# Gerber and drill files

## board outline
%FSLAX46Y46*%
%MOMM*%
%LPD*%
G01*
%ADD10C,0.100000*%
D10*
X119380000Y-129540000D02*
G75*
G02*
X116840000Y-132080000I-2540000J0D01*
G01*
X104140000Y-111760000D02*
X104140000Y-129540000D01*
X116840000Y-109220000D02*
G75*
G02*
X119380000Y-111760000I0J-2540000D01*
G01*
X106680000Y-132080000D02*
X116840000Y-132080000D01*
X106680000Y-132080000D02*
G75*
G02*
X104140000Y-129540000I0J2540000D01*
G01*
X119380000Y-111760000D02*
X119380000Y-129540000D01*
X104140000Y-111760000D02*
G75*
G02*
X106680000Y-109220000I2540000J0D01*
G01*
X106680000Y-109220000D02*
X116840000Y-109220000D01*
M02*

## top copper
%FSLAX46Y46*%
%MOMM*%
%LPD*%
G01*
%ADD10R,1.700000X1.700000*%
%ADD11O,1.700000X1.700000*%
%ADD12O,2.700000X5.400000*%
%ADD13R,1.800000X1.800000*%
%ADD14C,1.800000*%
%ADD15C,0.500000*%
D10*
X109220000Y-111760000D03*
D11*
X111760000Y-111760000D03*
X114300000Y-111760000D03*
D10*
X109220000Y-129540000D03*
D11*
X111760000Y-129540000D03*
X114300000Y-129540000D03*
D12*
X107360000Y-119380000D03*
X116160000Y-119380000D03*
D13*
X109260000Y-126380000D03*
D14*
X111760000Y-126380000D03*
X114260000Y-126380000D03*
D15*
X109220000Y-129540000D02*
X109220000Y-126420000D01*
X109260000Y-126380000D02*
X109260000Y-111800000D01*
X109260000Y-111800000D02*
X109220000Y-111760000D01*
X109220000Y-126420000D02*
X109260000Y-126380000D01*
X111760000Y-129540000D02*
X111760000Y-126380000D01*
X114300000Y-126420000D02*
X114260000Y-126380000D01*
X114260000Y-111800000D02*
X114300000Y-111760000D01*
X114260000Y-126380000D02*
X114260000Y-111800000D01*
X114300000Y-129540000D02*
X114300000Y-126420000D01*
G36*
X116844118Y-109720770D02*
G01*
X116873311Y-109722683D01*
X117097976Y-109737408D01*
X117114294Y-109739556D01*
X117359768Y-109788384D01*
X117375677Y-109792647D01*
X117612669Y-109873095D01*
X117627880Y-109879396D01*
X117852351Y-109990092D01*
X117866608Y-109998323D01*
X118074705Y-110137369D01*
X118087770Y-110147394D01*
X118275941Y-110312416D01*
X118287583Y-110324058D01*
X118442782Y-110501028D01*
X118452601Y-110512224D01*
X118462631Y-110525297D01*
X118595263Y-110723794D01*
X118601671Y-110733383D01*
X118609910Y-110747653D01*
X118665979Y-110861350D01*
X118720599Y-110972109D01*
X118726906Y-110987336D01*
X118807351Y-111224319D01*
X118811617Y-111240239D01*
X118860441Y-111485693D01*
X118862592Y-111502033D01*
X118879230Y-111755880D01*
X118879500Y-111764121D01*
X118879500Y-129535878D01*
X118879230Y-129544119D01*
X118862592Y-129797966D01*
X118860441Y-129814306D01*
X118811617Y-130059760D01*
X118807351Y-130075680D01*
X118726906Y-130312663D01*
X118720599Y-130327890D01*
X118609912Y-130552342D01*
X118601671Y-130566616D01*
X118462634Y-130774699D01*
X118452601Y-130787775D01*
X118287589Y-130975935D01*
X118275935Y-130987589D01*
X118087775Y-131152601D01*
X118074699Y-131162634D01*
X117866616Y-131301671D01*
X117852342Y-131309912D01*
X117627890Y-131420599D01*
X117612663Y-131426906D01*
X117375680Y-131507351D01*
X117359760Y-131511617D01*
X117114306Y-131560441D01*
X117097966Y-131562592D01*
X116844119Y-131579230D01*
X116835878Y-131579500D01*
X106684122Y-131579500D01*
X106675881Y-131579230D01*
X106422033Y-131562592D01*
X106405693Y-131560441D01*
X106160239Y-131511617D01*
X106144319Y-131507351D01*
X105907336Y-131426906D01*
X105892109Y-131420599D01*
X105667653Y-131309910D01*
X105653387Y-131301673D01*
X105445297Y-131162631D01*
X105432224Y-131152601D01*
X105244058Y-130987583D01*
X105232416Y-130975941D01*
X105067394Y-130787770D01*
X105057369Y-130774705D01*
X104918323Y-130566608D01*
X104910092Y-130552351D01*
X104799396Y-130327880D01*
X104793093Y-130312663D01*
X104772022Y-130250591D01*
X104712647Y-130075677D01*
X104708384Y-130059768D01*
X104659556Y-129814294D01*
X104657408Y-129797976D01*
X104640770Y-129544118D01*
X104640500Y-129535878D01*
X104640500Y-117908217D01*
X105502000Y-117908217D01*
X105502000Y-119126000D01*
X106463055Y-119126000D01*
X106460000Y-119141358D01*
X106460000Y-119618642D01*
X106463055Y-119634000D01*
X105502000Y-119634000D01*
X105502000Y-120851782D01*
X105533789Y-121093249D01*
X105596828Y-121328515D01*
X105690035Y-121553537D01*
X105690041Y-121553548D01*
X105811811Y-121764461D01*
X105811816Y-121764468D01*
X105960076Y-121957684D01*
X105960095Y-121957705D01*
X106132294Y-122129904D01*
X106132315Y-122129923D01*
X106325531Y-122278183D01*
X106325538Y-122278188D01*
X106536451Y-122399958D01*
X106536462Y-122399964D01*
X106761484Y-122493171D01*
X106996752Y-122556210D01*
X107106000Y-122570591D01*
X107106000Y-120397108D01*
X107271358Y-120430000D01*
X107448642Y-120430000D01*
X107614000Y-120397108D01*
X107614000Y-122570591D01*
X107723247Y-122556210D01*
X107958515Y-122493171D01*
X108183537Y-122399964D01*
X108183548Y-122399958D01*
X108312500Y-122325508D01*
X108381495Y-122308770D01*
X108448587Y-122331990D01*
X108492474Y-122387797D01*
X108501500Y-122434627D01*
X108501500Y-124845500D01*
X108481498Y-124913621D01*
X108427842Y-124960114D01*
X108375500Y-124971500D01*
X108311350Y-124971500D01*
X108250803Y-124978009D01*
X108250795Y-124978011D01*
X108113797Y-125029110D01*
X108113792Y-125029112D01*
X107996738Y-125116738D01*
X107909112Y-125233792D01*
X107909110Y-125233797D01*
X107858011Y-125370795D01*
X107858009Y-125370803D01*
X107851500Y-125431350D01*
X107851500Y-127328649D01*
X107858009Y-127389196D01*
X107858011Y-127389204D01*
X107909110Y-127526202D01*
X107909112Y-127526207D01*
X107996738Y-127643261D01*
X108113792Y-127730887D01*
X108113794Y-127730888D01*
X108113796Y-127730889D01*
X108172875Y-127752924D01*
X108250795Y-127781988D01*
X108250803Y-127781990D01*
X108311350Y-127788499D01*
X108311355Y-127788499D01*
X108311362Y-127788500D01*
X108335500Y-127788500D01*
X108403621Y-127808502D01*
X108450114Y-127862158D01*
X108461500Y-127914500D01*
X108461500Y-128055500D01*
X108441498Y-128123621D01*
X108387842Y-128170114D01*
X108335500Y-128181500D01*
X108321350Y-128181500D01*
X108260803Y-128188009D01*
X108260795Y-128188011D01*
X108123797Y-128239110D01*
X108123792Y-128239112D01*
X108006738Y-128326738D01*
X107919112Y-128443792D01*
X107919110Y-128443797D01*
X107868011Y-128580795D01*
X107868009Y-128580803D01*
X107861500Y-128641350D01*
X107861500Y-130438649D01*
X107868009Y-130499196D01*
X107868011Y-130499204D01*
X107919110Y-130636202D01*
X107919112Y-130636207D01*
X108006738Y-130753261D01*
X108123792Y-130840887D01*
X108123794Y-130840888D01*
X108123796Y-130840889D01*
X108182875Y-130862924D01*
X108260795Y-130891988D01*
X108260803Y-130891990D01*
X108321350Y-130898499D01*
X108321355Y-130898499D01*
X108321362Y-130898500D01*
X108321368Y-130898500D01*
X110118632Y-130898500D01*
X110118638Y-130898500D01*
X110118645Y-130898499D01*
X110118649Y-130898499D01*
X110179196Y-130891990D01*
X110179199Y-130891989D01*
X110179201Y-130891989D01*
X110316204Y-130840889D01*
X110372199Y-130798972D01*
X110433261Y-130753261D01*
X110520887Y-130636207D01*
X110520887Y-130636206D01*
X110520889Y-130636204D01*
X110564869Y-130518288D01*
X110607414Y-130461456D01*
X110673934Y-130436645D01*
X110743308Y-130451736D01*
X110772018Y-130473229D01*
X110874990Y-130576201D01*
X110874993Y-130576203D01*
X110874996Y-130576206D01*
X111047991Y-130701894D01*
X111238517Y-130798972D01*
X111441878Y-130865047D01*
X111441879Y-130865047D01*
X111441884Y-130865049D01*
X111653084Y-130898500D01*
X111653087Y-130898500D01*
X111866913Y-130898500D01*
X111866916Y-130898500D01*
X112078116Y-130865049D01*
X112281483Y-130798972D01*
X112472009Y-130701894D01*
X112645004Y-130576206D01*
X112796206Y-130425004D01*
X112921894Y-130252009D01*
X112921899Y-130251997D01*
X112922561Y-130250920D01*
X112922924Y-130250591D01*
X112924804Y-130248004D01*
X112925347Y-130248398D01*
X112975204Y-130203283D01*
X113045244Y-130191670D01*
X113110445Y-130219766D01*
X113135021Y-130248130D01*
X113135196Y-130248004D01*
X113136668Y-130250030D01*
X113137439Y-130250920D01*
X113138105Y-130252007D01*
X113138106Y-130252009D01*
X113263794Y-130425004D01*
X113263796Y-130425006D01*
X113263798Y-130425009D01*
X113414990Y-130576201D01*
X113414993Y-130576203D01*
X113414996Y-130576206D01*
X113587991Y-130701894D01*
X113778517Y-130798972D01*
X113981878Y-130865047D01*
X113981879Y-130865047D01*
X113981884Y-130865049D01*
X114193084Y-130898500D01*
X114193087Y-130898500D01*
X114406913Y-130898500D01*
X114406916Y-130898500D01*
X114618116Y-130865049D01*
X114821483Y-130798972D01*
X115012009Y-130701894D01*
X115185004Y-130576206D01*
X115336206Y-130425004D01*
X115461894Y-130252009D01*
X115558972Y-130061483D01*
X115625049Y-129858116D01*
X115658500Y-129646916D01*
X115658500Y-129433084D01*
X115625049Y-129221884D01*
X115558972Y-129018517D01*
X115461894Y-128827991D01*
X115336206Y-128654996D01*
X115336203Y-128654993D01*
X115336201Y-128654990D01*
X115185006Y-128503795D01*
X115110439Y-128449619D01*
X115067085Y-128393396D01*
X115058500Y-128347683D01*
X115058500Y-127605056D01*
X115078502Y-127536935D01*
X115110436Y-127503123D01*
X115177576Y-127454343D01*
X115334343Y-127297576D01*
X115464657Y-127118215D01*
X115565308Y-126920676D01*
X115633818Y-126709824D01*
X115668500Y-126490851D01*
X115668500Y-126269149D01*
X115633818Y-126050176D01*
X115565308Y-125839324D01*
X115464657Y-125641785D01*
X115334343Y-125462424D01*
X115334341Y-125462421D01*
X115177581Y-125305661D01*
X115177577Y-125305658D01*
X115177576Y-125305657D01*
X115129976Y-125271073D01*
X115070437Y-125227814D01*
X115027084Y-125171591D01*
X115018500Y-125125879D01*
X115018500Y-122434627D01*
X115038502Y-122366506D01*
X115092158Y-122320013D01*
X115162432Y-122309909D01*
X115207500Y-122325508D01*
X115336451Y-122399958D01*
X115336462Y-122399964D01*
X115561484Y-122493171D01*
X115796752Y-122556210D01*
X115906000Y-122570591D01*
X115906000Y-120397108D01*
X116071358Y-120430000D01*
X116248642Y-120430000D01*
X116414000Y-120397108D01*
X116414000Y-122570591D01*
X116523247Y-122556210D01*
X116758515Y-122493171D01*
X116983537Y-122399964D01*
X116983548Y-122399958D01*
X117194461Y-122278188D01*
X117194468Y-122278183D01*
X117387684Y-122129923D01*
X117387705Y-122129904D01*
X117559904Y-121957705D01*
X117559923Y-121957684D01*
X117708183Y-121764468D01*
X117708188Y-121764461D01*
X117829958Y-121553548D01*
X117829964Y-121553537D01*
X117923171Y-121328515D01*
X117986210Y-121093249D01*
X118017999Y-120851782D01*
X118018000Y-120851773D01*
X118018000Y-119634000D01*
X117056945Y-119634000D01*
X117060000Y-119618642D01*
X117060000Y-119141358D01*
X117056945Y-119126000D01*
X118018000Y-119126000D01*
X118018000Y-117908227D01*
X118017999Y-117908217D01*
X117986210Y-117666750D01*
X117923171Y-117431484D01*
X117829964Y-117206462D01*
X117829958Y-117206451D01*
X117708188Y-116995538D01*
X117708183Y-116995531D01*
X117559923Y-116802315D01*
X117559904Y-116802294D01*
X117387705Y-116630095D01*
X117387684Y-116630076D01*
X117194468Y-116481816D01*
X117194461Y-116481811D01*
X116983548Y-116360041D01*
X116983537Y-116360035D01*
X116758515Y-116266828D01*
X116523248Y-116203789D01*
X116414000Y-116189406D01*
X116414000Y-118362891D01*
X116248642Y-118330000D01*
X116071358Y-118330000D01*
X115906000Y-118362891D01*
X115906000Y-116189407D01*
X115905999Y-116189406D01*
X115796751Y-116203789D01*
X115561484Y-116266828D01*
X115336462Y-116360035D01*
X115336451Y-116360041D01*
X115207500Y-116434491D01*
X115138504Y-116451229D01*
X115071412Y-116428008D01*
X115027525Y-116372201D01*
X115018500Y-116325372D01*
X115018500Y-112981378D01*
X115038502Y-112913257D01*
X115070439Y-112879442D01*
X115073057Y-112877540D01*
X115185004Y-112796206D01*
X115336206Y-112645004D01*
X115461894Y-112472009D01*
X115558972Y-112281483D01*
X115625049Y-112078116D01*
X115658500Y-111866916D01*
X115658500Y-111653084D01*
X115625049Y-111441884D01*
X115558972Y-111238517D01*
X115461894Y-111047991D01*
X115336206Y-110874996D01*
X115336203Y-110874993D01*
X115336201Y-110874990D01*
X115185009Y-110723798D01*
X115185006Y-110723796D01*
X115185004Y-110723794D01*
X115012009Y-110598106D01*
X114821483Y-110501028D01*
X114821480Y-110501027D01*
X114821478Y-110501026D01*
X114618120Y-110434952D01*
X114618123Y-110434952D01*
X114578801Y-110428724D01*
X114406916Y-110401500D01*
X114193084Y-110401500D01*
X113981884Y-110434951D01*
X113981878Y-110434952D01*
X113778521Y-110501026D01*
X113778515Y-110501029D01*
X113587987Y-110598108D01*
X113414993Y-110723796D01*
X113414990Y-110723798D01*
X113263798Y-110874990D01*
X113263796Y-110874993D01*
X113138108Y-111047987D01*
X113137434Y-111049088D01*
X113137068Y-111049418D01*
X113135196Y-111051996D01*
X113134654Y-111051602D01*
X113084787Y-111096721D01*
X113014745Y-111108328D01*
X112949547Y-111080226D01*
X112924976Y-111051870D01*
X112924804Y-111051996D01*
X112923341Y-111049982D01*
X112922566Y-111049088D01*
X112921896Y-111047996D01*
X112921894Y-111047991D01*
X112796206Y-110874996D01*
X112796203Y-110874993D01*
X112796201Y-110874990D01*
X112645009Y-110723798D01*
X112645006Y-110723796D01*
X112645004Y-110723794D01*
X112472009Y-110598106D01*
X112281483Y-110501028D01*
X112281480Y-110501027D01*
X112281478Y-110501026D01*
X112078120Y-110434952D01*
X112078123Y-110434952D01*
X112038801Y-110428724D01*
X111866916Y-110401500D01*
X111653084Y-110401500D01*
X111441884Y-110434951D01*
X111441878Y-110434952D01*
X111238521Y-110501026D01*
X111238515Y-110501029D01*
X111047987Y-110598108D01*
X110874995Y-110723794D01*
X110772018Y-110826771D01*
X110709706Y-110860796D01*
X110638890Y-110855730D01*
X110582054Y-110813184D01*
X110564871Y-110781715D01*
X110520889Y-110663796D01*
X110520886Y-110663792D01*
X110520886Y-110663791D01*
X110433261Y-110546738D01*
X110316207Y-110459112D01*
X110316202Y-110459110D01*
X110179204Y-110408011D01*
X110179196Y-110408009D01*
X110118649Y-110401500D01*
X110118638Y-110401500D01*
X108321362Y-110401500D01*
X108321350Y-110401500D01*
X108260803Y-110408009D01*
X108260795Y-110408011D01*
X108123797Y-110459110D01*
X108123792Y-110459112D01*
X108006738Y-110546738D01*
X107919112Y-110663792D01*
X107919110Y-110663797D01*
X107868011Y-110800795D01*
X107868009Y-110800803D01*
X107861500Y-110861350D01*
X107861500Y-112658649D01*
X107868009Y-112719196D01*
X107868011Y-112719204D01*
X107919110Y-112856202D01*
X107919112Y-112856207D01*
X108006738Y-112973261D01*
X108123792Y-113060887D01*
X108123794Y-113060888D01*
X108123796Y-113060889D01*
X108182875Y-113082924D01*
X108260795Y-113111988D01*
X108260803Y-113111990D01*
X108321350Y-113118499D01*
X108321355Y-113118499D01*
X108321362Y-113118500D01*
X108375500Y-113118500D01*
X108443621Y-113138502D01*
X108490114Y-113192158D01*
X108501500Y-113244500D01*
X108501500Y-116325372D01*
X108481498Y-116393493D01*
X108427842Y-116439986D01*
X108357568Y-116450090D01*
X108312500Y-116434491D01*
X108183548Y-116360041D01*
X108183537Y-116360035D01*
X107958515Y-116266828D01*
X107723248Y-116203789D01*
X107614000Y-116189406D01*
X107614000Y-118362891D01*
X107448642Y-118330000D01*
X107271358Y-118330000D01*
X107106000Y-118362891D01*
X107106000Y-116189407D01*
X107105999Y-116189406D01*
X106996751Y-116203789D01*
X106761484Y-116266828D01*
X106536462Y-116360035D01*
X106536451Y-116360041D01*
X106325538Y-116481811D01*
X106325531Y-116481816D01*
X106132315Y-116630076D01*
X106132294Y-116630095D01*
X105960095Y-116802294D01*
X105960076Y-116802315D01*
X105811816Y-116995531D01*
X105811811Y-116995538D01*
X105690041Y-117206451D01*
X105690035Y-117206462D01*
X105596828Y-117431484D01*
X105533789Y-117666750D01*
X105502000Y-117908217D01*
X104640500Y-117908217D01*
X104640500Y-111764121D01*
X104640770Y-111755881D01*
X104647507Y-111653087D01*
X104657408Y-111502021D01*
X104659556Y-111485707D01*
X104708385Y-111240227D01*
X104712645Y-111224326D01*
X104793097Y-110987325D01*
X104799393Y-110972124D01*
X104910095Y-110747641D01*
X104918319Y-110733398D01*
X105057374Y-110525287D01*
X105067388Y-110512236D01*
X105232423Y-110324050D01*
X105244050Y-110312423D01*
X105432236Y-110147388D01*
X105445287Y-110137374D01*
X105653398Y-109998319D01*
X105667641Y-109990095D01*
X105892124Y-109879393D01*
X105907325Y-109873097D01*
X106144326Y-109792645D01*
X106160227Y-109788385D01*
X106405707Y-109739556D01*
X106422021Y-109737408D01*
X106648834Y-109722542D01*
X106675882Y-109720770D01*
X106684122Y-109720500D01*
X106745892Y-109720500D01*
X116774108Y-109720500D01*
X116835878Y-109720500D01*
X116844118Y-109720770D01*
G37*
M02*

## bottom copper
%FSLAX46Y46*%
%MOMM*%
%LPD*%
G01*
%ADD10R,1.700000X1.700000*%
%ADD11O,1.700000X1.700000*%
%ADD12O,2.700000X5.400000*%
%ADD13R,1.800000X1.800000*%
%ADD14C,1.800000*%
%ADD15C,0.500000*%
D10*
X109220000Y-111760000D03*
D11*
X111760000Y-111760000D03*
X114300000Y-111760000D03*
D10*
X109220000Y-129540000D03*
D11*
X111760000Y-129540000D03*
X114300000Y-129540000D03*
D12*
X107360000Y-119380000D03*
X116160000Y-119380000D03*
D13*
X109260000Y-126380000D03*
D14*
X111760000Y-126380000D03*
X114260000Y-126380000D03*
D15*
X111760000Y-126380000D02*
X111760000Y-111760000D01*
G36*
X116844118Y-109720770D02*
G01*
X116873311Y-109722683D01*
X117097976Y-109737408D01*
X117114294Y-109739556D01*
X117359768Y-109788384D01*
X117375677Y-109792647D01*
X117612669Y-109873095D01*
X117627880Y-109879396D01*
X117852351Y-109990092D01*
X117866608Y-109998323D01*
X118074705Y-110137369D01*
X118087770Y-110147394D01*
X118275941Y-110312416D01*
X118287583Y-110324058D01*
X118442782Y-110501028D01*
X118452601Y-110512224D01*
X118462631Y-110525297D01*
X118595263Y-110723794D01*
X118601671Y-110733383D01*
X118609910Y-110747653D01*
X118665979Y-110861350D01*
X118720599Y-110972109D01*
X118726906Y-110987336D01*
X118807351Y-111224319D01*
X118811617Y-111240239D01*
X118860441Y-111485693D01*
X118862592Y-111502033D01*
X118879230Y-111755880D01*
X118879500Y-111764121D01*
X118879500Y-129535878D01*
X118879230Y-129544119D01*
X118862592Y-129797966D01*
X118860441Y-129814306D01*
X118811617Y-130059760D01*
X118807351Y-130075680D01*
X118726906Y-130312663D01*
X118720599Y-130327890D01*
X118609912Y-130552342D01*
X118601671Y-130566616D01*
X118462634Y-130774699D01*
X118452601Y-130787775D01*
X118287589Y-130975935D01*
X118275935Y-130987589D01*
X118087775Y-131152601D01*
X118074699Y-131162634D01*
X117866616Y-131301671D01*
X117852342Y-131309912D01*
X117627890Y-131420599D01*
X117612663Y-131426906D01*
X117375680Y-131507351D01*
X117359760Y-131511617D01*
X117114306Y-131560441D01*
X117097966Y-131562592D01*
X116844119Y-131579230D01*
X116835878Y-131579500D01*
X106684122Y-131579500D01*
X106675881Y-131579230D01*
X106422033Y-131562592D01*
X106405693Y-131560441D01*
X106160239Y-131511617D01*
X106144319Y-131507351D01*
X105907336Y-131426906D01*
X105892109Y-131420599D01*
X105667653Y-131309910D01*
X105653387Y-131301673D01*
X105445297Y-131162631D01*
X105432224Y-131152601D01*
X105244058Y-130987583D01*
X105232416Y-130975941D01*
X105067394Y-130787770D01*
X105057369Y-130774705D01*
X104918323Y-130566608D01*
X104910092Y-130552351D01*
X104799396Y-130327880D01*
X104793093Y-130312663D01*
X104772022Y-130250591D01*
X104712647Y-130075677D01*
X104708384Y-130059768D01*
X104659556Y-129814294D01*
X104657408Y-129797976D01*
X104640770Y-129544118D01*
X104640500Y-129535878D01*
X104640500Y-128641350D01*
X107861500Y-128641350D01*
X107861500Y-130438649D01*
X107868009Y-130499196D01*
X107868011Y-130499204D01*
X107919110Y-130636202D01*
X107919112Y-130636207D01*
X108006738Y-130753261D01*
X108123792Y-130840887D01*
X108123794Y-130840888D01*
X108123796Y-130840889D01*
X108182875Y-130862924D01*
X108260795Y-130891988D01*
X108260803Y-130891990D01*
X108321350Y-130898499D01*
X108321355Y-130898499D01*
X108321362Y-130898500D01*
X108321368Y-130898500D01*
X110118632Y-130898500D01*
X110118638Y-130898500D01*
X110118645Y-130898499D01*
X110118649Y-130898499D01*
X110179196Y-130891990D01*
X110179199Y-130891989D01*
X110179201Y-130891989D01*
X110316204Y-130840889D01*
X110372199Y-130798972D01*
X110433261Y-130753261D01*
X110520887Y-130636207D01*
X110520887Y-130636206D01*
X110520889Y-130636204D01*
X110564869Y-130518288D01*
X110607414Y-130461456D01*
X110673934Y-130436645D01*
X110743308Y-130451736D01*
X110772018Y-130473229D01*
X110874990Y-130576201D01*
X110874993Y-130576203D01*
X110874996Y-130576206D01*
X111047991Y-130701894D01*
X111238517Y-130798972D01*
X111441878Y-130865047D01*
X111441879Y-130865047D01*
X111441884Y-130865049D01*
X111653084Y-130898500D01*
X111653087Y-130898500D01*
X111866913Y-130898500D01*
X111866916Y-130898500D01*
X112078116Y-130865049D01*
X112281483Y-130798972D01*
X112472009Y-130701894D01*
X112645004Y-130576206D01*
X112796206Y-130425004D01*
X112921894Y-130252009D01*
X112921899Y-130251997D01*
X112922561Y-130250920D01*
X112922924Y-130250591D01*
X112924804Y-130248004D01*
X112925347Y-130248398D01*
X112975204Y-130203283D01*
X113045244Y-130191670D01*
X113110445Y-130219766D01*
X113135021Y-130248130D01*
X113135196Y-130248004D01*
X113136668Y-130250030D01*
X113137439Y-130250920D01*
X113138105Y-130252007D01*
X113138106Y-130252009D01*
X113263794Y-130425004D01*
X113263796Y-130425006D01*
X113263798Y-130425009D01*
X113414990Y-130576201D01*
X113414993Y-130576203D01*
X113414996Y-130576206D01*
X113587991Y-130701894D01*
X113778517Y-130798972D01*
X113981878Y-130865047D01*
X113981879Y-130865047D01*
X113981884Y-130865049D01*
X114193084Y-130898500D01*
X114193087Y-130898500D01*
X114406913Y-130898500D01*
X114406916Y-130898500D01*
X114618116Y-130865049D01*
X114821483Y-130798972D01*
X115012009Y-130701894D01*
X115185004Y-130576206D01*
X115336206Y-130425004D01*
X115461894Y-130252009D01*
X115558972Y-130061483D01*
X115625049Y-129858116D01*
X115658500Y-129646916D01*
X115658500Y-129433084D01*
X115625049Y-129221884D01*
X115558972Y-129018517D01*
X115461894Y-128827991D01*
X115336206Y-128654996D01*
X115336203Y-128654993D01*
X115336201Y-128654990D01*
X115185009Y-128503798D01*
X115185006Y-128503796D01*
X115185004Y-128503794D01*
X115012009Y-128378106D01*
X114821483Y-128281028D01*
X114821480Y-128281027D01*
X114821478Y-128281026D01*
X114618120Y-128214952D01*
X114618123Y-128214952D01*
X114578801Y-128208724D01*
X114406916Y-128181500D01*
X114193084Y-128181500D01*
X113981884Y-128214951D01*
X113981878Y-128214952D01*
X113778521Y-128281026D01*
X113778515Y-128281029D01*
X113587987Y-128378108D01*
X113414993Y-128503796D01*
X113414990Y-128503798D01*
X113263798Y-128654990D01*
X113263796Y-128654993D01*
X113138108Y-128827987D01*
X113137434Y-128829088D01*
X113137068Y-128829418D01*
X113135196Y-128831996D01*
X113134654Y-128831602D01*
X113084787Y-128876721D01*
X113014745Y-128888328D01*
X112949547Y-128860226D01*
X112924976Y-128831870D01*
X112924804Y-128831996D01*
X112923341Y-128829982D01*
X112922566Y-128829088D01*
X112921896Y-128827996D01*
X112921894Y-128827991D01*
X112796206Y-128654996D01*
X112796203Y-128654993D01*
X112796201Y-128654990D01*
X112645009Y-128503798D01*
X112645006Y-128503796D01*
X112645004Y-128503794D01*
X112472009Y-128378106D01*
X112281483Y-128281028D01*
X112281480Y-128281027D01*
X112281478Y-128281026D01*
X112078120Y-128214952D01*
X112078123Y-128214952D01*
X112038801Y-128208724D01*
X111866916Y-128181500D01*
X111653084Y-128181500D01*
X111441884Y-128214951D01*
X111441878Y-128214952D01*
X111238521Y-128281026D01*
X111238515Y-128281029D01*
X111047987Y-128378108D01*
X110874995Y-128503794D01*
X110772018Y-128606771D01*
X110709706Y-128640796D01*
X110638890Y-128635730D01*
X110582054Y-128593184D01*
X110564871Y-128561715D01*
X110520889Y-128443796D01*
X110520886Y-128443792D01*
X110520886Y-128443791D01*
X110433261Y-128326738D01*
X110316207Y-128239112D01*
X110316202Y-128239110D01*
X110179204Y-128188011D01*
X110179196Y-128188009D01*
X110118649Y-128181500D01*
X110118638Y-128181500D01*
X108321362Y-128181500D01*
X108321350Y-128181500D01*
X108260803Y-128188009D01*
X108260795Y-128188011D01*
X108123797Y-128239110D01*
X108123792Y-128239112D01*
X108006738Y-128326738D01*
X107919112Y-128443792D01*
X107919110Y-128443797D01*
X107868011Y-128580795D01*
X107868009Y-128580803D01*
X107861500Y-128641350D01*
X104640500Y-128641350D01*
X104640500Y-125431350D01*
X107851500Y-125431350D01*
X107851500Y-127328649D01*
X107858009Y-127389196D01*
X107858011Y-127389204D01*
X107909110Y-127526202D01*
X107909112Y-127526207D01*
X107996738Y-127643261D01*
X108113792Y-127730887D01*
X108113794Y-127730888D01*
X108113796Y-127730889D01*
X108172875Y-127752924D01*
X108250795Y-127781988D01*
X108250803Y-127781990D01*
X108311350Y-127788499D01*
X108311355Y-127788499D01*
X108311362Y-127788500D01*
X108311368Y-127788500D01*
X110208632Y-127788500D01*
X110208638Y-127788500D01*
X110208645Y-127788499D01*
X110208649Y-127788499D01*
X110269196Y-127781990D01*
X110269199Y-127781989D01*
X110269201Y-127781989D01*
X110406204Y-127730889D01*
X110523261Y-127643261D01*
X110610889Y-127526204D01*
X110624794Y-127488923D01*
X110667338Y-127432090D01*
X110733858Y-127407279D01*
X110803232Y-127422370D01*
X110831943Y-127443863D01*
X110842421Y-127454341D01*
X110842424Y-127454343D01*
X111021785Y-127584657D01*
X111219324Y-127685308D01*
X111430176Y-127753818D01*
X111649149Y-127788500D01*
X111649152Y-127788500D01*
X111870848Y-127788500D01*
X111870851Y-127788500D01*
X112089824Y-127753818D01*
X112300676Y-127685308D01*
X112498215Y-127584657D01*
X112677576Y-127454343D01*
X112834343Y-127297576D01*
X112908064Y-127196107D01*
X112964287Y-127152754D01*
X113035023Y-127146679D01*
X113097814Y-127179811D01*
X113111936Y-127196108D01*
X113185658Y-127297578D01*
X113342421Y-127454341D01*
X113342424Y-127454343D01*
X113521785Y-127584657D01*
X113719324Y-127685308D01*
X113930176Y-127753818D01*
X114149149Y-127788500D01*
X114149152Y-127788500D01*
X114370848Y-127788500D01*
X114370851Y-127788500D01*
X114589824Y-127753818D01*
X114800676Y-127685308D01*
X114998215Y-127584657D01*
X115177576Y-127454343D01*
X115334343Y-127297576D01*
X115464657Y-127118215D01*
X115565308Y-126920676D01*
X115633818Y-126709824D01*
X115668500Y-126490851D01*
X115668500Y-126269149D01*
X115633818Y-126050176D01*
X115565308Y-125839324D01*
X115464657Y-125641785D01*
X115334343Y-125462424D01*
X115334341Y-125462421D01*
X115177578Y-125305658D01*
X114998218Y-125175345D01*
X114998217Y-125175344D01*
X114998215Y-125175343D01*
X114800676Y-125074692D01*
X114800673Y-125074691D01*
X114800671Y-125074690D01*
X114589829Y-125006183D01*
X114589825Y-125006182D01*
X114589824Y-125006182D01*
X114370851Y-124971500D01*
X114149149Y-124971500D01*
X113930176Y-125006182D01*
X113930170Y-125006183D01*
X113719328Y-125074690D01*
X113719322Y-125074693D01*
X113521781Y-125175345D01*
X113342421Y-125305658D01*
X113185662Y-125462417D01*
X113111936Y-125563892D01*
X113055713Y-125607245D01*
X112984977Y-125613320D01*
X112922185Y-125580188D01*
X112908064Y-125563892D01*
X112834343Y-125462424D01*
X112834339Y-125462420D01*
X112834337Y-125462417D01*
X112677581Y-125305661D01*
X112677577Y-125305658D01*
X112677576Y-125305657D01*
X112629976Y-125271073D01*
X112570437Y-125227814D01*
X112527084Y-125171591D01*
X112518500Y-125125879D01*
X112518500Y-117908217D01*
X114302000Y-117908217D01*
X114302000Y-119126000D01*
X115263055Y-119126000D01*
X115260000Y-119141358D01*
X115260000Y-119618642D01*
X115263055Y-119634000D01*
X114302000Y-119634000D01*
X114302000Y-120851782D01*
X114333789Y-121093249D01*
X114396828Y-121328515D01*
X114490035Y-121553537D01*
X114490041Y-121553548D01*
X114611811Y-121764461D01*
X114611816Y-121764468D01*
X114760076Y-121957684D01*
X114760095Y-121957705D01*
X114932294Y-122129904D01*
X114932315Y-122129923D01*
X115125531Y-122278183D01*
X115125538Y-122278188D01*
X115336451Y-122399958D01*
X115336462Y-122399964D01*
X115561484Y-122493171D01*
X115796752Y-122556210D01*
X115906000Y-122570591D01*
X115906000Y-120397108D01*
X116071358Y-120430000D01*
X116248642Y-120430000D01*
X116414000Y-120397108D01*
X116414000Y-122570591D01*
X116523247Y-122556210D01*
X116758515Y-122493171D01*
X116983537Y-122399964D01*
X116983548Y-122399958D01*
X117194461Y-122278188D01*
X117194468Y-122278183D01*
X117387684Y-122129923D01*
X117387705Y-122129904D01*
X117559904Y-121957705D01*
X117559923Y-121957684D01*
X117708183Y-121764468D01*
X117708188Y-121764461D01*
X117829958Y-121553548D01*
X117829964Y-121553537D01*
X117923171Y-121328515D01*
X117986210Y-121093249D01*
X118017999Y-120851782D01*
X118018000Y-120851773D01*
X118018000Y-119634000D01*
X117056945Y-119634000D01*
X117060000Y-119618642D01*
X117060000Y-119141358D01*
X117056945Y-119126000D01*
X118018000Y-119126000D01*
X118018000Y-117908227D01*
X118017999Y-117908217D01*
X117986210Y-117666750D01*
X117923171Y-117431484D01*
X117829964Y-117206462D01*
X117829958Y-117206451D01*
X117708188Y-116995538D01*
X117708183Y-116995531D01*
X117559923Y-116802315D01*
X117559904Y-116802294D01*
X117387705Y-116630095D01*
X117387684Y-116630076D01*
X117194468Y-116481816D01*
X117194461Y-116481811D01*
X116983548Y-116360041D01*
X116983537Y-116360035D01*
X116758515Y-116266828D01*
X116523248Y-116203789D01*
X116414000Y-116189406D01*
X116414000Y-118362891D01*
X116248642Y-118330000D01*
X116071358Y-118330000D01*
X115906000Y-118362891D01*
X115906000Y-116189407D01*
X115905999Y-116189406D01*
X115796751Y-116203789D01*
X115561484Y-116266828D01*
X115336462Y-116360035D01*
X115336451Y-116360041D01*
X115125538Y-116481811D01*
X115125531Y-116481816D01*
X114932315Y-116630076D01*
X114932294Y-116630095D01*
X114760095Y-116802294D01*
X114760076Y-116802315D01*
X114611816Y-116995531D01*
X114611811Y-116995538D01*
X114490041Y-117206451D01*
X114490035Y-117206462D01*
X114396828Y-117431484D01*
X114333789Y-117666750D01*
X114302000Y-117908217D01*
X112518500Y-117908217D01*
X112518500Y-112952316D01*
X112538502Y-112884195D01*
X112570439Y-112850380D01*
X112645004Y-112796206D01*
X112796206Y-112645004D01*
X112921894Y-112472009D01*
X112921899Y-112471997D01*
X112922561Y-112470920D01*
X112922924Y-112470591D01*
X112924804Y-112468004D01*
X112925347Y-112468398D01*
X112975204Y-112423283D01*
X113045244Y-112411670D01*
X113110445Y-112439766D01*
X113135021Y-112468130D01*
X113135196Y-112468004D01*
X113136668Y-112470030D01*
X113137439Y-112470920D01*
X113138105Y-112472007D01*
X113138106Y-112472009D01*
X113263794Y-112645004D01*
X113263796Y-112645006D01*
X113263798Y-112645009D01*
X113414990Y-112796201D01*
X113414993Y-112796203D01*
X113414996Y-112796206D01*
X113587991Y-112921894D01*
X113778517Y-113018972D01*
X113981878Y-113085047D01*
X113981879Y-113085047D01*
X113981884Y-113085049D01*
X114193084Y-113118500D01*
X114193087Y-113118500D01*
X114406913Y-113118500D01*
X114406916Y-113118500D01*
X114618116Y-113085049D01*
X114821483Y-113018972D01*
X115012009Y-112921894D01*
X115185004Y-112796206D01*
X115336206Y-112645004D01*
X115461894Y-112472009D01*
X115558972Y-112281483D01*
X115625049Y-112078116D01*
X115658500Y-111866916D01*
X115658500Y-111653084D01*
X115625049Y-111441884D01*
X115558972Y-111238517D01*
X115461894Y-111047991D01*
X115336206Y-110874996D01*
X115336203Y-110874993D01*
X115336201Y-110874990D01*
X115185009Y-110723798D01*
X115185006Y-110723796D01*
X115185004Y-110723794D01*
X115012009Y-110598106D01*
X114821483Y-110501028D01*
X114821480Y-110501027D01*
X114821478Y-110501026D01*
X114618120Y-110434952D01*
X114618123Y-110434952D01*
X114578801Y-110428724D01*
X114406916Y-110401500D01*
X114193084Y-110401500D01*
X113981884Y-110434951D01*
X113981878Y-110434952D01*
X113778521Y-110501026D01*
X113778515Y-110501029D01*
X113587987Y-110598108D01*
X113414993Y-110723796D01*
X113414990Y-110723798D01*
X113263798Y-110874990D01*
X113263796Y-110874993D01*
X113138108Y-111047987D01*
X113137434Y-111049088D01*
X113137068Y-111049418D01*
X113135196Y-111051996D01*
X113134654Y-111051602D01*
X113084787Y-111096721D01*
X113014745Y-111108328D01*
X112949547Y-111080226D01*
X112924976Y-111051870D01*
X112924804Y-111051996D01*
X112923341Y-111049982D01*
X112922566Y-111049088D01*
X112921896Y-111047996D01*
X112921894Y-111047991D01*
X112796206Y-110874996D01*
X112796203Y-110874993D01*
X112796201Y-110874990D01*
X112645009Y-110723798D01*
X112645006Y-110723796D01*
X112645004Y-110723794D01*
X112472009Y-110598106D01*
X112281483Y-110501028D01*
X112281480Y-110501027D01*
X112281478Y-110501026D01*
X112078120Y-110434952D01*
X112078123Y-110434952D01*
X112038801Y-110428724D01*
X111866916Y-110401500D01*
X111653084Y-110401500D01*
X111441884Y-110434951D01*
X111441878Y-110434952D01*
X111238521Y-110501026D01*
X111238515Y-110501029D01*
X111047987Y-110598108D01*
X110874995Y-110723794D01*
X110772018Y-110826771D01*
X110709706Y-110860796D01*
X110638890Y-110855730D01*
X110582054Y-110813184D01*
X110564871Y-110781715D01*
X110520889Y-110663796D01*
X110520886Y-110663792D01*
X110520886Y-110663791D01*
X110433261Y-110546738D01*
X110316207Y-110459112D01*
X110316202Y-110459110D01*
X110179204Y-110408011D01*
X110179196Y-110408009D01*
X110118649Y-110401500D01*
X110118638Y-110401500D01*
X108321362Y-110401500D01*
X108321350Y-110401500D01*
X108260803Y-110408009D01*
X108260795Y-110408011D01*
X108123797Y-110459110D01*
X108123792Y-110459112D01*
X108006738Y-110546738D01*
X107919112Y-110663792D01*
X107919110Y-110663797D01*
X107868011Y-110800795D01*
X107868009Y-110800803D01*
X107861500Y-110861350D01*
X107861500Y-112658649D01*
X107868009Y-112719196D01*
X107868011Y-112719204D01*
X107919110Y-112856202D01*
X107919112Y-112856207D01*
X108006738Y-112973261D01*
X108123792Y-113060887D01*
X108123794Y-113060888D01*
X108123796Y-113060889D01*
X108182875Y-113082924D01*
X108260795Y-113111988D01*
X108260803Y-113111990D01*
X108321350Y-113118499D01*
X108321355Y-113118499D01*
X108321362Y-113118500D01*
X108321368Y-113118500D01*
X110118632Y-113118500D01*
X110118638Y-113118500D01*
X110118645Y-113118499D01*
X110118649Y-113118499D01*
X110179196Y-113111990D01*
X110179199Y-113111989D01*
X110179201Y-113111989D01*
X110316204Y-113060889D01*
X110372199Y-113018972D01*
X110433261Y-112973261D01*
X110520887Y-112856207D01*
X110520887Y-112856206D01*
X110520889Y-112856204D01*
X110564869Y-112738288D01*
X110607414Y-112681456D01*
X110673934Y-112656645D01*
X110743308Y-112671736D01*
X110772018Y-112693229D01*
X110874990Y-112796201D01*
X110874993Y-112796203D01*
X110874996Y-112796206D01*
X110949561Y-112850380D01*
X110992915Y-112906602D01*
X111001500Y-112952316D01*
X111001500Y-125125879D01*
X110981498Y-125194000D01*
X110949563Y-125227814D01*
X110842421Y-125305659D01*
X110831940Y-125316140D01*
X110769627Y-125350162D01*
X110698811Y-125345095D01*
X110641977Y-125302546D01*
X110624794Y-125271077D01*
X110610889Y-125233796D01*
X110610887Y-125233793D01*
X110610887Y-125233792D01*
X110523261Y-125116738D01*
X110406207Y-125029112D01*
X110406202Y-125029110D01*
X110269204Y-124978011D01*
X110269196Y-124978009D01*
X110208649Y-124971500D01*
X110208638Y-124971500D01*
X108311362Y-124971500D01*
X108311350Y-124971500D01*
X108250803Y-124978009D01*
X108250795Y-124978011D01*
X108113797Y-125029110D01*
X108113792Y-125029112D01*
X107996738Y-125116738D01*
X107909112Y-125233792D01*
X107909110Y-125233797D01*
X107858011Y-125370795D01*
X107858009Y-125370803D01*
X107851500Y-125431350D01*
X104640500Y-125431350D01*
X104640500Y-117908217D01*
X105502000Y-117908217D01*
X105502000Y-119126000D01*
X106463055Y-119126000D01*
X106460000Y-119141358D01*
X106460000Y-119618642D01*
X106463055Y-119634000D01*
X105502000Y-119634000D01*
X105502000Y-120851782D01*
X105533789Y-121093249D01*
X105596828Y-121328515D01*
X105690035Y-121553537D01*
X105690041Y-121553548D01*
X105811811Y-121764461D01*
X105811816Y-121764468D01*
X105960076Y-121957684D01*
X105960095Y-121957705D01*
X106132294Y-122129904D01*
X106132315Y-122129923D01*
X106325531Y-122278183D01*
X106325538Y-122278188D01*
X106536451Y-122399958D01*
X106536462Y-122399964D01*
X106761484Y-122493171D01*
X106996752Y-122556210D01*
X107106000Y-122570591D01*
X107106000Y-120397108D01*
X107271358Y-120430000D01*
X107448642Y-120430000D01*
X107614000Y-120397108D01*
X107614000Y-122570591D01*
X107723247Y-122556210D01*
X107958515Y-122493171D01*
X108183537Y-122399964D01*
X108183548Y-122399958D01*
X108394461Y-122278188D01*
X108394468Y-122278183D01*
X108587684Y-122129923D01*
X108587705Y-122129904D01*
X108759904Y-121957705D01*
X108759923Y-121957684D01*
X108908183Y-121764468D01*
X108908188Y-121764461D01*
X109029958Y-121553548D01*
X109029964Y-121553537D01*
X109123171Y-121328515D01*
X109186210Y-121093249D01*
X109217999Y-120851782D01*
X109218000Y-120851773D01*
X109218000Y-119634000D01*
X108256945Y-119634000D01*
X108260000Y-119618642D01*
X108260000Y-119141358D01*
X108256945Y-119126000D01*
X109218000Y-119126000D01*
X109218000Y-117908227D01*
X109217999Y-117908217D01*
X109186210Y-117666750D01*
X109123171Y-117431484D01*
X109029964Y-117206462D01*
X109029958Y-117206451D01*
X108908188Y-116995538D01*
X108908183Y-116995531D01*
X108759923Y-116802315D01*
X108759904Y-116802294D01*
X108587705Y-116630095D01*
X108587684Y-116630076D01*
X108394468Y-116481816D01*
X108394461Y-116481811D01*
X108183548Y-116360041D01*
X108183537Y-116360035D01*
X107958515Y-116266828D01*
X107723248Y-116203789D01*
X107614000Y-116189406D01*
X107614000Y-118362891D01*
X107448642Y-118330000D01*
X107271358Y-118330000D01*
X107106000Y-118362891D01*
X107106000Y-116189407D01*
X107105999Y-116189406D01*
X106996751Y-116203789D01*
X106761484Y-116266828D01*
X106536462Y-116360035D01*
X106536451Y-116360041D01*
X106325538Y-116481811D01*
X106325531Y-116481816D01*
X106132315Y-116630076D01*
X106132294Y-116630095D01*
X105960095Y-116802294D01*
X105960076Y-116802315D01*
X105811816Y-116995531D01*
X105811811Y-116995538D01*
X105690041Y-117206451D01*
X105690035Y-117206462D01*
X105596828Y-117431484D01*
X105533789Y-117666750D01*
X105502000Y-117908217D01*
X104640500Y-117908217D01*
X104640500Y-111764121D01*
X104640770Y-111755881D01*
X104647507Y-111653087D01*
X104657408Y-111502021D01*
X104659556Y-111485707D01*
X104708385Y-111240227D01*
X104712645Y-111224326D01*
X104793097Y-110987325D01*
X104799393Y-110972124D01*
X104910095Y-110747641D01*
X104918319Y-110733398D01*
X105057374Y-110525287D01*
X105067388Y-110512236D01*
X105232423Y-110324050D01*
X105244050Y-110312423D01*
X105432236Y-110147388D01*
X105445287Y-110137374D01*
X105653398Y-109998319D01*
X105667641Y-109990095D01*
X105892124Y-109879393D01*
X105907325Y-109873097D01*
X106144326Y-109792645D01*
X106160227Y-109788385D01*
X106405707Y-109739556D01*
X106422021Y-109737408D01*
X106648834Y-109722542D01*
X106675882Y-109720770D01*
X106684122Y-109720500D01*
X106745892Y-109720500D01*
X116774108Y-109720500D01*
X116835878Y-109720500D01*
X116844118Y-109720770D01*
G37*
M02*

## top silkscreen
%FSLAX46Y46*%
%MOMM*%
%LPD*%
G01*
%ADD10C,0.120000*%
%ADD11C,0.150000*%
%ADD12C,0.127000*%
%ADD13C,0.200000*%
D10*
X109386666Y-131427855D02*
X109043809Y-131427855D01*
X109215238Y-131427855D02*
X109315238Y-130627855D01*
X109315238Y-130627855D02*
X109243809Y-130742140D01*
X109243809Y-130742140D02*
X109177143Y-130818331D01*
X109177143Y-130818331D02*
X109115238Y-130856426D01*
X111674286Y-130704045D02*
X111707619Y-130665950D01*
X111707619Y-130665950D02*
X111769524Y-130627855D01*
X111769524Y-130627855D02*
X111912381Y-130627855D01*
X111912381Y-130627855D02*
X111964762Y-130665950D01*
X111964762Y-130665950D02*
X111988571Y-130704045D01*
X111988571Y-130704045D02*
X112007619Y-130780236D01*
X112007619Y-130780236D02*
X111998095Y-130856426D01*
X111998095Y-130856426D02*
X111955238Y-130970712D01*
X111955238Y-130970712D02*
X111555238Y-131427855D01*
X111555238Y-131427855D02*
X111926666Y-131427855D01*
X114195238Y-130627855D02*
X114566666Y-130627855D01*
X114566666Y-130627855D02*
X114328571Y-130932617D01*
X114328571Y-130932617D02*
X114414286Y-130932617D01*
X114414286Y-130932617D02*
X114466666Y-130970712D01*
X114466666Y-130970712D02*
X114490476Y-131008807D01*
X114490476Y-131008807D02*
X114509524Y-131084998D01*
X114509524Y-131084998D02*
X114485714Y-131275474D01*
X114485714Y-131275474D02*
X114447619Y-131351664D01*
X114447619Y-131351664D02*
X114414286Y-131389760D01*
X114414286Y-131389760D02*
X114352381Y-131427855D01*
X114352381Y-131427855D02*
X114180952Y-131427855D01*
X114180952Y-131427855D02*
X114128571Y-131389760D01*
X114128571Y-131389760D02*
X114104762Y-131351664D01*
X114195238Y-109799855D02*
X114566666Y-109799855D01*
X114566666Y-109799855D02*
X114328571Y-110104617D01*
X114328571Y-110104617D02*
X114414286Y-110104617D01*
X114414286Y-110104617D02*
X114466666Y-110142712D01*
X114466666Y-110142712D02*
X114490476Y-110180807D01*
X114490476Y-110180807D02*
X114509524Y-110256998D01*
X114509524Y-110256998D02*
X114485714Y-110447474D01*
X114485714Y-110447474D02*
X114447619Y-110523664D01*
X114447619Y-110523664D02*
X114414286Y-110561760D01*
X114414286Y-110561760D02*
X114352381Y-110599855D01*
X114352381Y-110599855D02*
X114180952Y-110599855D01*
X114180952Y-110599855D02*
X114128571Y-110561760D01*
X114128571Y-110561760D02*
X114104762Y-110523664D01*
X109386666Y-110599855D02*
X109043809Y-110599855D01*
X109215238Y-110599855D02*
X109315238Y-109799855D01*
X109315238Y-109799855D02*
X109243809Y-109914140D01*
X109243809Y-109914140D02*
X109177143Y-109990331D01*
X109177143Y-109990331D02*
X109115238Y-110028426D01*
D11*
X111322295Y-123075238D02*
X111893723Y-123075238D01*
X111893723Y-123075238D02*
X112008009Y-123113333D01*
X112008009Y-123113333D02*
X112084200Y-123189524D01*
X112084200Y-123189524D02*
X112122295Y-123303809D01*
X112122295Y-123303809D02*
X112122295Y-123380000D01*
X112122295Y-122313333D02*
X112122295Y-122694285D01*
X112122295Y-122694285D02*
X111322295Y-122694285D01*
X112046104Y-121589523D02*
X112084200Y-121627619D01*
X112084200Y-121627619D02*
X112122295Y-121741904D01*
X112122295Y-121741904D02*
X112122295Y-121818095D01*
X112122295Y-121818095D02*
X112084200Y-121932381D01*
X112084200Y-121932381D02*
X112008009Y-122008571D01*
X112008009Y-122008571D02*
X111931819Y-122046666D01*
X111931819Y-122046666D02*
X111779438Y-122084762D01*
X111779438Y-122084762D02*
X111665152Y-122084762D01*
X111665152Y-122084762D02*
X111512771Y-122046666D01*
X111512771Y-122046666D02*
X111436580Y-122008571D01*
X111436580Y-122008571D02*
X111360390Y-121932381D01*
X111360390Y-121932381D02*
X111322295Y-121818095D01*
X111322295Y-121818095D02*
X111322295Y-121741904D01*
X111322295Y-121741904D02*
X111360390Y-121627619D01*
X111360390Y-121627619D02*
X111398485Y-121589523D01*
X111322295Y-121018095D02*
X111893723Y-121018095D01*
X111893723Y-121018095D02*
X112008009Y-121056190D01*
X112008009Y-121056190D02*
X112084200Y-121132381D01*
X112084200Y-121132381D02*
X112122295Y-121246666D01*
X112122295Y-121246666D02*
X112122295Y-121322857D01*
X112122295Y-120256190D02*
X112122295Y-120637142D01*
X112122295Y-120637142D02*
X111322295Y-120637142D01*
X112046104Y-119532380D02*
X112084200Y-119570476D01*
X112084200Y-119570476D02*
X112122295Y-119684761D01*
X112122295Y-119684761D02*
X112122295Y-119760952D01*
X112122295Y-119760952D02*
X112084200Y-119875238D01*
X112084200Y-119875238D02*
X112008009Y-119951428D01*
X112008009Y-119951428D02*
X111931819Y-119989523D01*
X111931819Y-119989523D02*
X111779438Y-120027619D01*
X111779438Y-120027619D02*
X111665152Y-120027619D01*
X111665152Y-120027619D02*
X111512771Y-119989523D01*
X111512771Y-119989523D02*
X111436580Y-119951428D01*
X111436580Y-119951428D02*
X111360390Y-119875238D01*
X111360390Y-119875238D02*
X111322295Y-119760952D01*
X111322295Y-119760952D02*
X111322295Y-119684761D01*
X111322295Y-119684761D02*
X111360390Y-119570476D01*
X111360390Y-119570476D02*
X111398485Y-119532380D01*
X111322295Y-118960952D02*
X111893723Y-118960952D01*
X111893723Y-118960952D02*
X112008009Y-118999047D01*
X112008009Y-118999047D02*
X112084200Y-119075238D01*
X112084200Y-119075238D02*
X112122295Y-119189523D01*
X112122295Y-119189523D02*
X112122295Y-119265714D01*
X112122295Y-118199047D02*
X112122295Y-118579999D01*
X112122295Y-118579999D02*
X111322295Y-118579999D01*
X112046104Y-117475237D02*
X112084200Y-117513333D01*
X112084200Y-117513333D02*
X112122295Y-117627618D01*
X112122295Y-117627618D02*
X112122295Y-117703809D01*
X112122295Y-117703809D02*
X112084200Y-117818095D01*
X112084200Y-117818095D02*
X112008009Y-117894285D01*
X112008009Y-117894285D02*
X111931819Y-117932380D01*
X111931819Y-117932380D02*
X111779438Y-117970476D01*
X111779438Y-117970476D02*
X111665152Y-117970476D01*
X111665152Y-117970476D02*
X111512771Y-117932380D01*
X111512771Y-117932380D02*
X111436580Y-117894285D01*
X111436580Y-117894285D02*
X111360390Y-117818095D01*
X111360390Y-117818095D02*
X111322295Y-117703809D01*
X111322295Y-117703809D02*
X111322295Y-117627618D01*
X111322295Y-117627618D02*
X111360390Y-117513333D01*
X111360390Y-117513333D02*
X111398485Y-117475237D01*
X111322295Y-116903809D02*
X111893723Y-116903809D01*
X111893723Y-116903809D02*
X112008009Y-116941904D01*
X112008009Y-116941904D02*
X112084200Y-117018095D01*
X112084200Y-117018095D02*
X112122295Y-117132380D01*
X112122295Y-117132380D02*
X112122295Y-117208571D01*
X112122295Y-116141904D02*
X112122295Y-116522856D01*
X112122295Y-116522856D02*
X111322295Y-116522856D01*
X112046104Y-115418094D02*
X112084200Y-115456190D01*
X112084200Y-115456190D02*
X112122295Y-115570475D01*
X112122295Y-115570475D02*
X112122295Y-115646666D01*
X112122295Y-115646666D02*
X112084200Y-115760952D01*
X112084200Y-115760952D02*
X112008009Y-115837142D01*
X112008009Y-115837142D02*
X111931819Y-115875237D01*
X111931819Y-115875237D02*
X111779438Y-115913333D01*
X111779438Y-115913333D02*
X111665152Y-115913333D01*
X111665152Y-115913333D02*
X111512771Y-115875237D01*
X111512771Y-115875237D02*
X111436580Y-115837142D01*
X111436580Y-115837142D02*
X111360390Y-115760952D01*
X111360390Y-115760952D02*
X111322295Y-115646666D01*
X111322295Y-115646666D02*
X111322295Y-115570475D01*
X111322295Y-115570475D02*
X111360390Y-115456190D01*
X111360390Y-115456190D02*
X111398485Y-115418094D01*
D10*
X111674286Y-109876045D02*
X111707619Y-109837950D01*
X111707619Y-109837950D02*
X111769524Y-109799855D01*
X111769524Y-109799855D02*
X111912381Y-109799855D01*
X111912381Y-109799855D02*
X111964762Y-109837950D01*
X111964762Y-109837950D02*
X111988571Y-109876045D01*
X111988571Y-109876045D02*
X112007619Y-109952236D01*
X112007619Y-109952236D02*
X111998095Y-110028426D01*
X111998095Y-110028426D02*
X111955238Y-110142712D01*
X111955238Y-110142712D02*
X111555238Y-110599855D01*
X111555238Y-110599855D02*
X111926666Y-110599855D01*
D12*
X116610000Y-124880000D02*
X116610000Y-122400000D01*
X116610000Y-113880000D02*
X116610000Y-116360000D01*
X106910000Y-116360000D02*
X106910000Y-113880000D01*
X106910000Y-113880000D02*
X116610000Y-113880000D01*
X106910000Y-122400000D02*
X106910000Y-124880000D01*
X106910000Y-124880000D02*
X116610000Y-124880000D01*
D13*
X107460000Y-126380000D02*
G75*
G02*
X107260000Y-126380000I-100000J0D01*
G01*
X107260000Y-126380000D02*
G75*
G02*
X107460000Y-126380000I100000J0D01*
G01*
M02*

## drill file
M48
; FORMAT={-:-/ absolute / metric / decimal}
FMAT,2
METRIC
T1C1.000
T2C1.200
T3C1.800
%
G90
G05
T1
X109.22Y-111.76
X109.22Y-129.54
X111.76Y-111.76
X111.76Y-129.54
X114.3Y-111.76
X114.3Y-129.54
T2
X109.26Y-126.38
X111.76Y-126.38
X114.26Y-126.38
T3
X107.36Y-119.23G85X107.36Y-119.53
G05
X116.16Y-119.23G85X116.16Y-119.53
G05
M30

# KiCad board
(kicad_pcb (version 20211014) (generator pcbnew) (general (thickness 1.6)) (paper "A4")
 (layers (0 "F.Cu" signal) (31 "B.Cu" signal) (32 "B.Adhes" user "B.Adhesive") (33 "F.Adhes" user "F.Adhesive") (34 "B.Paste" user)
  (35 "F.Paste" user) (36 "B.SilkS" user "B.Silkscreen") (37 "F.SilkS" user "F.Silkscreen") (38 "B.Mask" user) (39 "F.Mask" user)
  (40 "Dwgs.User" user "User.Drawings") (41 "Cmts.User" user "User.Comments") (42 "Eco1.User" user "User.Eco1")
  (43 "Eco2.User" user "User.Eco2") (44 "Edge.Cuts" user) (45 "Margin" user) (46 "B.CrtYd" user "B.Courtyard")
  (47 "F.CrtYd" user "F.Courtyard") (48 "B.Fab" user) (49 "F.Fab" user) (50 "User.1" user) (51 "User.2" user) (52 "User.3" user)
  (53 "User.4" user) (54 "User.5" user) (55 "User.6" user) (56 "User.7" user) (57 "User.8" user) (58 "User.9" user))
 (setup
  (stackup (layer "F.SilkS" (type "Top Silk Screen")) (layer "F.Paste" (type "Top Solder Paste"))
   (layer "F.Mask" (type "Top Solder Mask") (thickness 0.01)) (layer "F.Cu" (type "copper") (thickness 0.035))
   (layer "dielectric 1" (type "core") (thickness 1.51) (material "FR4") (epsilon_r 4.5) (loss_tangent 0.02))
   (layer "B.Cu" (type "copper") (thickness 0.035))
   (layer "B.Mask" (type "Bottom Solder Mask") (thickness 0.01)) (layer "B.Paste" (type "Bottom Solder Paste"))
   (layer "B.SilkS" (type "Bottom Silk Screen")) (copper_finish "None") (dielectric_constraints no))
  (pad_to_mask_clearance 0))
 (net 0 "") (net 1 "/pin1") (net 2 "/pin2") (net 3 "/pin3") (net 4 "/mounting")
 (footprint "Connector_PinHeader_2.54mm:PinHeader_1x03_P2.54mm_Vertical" (layer "F.Cu") (at 109.22 111.76 90)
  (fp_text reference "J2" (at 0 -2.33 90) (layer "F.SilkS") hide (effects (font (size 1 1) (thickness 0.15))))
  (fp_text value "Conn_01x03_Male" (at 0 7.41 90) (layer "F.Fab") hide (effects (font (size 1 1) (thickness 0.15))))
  (pad "1" thru_hole rect (at 0 0 90) (size 1.7 1.7) (drill 1) (layers *.Cu *.Mask) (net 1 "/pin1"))
  (pad "2" thru_hole oval (at 0 2.54 90) (size 1.7 1.7) (drill 1) (layers *.Cu *.Mask) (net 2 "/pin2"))
  (pad "3" thru_hole oval (at 0 5.08 90) (size 1.7 1.7) (drill 1) (layers *.Cu *.Mask) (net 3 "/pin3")))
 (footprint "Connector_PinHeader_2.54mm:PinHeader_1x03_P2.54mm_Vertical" (layer "F.Cu") (at 109.22 129.54 90)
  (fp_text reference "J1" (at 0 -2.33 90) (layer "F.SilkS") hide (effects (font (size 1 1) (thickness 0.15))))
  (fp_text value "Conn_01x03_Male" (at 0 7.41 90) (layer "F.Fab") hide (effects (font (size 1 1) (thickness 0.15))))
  (pad "1" thru_hole rect (at 0 0 90) (size 1.7 1.7) (drill 1) (layers *.Cu *.Mask) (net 1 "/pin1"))
  (pad "2" thru_hole oval (at 0 2.54 90) (size 1.7 1.7) (drill 1) (layers *.Cu *.Mask) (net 2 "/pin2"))
  (pad "3" thru_hole oval (at 0 5.08 90) (size 1.7 1.7) (drill 1) (layers *.Cu *.Mask) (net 3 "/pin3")))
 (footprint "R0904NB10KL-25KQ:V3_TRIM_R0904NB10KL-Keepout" (layer "F.Cu") (at 111.76 119.38)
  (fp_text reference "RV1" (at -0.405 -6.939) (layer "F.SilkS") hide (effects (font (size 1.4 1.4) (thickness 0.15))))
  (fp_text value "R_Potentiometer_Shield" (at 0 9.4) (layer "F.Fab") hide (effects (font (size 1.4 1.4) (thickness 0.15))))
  (fp_line (start 4.85 5.5) (end 4.85 3.02) (layer "F.SilkS") (width 0.127))
  (fp_line (start 4.85 -5.5) (end 4.85 -3.02) (layer "F.SilkS") (width 0.127))
  (fp_line (start -4.85 -3.02) (end -4.85 -5.5) (layer "F.SilkS") (width 0.127))
  (fp_line (start -4.85 -5.5) (end 4.85 -5.5) (layer "F.SilkS") (width 0.127))
  (fp_line (start -4.85 3.02) (end -4.85 5.5) (layer "F.SilkS") (width 0.127))
  (fp_line (start -4.85 5.5) (end 4.85 5.5) (layer "F.SilkS") (width 0.127))
  (fp_circle (center -4.4 7) (end -4.3 7) (layer "F.SilkS") (width 0.2) (fill none))
  (pad "0" thru_hole oval (at -4.4 0) (size 2.7 5.4) (drill oval 1.8 2.1) (layers *.Cu *.Mask) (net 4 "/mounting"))
  (pad "0" thru_hole oval (at 4.4 0) (size 2.7 5.4) (drill oval 1.8 2.1) (layers *.Cu *.Mask) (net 4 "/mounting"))
  (pad "1" thru_hole rect (at -2.5 7) (size 1.8 1.8) (drill 1.2) (layers *.Cu *.Mask) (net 1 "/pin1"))
  (pad "2" thru_hole circle (at 0 7) (size 1.8 1.8) (drill 1.2) (layers *.Cu *.Mask) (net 2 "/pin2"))
  (pad "3" thru_hole circle (at 2.5 7) (size 1.8 1.8) (drill 1.2) (layers *.Cu *.Mask) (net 3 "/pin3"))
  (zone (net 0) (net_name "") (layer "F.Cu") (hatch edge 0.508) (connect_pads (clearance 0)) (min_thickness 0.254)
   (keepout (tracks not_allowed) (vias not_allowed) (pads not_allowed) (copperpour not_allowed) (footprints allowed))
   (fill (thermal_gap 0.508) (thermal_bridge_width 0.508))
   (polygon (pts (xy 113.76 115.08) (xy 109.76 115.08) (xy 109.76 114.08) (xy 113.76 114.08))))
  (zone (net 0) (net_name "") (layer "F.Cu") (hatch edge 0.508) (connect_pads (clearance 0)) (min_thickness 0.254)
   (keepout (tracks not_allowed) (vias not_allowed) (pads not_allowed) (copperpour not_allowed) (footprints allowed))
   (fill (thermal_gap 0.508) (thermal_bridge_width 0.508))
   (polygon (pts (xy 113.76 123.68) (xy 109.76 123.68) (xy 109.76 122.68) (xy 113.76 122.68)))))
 (gr_arc (start 119.38 129.54) (mid 118.636051 131.336051) (end 116.84 132.08) (layer "Edge.Cuts") (width 0.1))
 (gr_line (start 104.14 111.76) (end 104.14 129.54) (layer "Edge.Cuts") (width 0.1))
 (gr_arc (start 116.84 109.22) (mid 118.636051 109.963949) (end 119.38 111.76) (layer "Edge.Cuts") (width 0.1))
 (gr_line (start 106.68 132.08) (end 116.84 132.08) (layer "Edge.Cuts") (width 0.1))
 (gr_arc (start 106.68 132.08) (mid 104.883949 131.336051) (end 104.14 129.54) (layer "Edge.Cuts") (width 0.1))
 (gr_line (start 119.38 111.76) (end 119.38 129.54) (layer "Edge.Cuts") (width 0.1))
 (gr_arc (start 104.14 111.76) (mid 104.883949 109.963949) (end 106.68 109.22) (layer "Edge.Cuts") (width 0.1))
 (gr_line (start 106.68 109.22) (end 116.84 109.22) (layer "Edge.Cuts") (width 0.1))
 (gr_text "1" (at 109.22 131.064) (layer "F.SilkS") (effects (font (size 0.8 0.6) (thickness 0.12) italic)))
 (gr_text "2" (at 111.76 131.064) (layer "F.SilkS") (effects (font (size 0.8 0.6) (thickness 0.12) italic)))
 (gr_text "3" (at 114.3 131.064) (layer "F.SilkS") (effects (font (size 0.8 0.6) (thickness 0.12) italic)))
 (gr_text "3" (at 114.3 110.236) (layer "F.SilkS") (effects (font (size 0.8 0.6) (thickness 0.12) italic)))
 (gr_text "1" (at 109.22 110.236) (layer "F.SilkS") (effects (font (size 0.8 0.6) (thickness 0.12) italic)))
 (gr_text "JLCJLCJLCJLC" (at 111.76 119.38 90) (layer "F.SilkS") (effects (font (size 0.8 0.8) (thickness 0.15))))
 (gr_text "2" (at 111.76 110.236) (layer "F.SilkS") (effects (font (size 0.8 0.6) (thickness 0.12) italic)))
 (segment (start 109.22 129.54) (end 109.22 126.42) (width 0.5) (layer "F.Cu") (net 1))
 (segment (start 109.26 126.38) (end 109.26 111.8) (width 0.5) (layer "F.Cu") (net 1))
 (segment (start 109.26 111.8) (end 109.22 111.76) (width 0.5) (layer "F.Cu") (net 1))
 (segment (start 109.22 126.42) (end 109.26 126.38) (width 0.5) (layer "F.Cu") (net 1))
 (segment (start 111.76 129.54) (end 111.76 126.38) (width 0.5) (layer "F.Cu") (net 2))
 (segment (start 111.76 126.38) (end 111.76 111.76) (width 0.5) (layer "B.Cu") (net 2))
 (segment (start 114.3 126.42) (end 114.26 126.38) (width 0.5) (layer "F.Cu") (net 3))
 (segment (start 114.26 111.8) (end 114.3 111.76) (width 0.5) (layer "F.Cu") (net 3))
 (segment (start 114.26 126.38) (end 114.26 111.8) (width 0.5) (layer "F.Cu") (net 3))
 (segment (start 114.3 129.54) (end 114.3 126.42) (width 0.5) (layer "F.Cu") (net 3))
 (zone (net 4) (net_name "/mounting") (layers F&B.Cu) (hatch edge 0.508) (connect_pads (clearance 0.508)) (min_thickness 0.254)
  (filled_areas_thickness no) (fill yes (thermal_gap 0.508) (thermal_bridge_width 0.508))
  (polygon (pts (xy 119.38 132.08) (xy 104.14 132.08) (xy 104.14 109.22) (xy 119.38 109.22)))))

